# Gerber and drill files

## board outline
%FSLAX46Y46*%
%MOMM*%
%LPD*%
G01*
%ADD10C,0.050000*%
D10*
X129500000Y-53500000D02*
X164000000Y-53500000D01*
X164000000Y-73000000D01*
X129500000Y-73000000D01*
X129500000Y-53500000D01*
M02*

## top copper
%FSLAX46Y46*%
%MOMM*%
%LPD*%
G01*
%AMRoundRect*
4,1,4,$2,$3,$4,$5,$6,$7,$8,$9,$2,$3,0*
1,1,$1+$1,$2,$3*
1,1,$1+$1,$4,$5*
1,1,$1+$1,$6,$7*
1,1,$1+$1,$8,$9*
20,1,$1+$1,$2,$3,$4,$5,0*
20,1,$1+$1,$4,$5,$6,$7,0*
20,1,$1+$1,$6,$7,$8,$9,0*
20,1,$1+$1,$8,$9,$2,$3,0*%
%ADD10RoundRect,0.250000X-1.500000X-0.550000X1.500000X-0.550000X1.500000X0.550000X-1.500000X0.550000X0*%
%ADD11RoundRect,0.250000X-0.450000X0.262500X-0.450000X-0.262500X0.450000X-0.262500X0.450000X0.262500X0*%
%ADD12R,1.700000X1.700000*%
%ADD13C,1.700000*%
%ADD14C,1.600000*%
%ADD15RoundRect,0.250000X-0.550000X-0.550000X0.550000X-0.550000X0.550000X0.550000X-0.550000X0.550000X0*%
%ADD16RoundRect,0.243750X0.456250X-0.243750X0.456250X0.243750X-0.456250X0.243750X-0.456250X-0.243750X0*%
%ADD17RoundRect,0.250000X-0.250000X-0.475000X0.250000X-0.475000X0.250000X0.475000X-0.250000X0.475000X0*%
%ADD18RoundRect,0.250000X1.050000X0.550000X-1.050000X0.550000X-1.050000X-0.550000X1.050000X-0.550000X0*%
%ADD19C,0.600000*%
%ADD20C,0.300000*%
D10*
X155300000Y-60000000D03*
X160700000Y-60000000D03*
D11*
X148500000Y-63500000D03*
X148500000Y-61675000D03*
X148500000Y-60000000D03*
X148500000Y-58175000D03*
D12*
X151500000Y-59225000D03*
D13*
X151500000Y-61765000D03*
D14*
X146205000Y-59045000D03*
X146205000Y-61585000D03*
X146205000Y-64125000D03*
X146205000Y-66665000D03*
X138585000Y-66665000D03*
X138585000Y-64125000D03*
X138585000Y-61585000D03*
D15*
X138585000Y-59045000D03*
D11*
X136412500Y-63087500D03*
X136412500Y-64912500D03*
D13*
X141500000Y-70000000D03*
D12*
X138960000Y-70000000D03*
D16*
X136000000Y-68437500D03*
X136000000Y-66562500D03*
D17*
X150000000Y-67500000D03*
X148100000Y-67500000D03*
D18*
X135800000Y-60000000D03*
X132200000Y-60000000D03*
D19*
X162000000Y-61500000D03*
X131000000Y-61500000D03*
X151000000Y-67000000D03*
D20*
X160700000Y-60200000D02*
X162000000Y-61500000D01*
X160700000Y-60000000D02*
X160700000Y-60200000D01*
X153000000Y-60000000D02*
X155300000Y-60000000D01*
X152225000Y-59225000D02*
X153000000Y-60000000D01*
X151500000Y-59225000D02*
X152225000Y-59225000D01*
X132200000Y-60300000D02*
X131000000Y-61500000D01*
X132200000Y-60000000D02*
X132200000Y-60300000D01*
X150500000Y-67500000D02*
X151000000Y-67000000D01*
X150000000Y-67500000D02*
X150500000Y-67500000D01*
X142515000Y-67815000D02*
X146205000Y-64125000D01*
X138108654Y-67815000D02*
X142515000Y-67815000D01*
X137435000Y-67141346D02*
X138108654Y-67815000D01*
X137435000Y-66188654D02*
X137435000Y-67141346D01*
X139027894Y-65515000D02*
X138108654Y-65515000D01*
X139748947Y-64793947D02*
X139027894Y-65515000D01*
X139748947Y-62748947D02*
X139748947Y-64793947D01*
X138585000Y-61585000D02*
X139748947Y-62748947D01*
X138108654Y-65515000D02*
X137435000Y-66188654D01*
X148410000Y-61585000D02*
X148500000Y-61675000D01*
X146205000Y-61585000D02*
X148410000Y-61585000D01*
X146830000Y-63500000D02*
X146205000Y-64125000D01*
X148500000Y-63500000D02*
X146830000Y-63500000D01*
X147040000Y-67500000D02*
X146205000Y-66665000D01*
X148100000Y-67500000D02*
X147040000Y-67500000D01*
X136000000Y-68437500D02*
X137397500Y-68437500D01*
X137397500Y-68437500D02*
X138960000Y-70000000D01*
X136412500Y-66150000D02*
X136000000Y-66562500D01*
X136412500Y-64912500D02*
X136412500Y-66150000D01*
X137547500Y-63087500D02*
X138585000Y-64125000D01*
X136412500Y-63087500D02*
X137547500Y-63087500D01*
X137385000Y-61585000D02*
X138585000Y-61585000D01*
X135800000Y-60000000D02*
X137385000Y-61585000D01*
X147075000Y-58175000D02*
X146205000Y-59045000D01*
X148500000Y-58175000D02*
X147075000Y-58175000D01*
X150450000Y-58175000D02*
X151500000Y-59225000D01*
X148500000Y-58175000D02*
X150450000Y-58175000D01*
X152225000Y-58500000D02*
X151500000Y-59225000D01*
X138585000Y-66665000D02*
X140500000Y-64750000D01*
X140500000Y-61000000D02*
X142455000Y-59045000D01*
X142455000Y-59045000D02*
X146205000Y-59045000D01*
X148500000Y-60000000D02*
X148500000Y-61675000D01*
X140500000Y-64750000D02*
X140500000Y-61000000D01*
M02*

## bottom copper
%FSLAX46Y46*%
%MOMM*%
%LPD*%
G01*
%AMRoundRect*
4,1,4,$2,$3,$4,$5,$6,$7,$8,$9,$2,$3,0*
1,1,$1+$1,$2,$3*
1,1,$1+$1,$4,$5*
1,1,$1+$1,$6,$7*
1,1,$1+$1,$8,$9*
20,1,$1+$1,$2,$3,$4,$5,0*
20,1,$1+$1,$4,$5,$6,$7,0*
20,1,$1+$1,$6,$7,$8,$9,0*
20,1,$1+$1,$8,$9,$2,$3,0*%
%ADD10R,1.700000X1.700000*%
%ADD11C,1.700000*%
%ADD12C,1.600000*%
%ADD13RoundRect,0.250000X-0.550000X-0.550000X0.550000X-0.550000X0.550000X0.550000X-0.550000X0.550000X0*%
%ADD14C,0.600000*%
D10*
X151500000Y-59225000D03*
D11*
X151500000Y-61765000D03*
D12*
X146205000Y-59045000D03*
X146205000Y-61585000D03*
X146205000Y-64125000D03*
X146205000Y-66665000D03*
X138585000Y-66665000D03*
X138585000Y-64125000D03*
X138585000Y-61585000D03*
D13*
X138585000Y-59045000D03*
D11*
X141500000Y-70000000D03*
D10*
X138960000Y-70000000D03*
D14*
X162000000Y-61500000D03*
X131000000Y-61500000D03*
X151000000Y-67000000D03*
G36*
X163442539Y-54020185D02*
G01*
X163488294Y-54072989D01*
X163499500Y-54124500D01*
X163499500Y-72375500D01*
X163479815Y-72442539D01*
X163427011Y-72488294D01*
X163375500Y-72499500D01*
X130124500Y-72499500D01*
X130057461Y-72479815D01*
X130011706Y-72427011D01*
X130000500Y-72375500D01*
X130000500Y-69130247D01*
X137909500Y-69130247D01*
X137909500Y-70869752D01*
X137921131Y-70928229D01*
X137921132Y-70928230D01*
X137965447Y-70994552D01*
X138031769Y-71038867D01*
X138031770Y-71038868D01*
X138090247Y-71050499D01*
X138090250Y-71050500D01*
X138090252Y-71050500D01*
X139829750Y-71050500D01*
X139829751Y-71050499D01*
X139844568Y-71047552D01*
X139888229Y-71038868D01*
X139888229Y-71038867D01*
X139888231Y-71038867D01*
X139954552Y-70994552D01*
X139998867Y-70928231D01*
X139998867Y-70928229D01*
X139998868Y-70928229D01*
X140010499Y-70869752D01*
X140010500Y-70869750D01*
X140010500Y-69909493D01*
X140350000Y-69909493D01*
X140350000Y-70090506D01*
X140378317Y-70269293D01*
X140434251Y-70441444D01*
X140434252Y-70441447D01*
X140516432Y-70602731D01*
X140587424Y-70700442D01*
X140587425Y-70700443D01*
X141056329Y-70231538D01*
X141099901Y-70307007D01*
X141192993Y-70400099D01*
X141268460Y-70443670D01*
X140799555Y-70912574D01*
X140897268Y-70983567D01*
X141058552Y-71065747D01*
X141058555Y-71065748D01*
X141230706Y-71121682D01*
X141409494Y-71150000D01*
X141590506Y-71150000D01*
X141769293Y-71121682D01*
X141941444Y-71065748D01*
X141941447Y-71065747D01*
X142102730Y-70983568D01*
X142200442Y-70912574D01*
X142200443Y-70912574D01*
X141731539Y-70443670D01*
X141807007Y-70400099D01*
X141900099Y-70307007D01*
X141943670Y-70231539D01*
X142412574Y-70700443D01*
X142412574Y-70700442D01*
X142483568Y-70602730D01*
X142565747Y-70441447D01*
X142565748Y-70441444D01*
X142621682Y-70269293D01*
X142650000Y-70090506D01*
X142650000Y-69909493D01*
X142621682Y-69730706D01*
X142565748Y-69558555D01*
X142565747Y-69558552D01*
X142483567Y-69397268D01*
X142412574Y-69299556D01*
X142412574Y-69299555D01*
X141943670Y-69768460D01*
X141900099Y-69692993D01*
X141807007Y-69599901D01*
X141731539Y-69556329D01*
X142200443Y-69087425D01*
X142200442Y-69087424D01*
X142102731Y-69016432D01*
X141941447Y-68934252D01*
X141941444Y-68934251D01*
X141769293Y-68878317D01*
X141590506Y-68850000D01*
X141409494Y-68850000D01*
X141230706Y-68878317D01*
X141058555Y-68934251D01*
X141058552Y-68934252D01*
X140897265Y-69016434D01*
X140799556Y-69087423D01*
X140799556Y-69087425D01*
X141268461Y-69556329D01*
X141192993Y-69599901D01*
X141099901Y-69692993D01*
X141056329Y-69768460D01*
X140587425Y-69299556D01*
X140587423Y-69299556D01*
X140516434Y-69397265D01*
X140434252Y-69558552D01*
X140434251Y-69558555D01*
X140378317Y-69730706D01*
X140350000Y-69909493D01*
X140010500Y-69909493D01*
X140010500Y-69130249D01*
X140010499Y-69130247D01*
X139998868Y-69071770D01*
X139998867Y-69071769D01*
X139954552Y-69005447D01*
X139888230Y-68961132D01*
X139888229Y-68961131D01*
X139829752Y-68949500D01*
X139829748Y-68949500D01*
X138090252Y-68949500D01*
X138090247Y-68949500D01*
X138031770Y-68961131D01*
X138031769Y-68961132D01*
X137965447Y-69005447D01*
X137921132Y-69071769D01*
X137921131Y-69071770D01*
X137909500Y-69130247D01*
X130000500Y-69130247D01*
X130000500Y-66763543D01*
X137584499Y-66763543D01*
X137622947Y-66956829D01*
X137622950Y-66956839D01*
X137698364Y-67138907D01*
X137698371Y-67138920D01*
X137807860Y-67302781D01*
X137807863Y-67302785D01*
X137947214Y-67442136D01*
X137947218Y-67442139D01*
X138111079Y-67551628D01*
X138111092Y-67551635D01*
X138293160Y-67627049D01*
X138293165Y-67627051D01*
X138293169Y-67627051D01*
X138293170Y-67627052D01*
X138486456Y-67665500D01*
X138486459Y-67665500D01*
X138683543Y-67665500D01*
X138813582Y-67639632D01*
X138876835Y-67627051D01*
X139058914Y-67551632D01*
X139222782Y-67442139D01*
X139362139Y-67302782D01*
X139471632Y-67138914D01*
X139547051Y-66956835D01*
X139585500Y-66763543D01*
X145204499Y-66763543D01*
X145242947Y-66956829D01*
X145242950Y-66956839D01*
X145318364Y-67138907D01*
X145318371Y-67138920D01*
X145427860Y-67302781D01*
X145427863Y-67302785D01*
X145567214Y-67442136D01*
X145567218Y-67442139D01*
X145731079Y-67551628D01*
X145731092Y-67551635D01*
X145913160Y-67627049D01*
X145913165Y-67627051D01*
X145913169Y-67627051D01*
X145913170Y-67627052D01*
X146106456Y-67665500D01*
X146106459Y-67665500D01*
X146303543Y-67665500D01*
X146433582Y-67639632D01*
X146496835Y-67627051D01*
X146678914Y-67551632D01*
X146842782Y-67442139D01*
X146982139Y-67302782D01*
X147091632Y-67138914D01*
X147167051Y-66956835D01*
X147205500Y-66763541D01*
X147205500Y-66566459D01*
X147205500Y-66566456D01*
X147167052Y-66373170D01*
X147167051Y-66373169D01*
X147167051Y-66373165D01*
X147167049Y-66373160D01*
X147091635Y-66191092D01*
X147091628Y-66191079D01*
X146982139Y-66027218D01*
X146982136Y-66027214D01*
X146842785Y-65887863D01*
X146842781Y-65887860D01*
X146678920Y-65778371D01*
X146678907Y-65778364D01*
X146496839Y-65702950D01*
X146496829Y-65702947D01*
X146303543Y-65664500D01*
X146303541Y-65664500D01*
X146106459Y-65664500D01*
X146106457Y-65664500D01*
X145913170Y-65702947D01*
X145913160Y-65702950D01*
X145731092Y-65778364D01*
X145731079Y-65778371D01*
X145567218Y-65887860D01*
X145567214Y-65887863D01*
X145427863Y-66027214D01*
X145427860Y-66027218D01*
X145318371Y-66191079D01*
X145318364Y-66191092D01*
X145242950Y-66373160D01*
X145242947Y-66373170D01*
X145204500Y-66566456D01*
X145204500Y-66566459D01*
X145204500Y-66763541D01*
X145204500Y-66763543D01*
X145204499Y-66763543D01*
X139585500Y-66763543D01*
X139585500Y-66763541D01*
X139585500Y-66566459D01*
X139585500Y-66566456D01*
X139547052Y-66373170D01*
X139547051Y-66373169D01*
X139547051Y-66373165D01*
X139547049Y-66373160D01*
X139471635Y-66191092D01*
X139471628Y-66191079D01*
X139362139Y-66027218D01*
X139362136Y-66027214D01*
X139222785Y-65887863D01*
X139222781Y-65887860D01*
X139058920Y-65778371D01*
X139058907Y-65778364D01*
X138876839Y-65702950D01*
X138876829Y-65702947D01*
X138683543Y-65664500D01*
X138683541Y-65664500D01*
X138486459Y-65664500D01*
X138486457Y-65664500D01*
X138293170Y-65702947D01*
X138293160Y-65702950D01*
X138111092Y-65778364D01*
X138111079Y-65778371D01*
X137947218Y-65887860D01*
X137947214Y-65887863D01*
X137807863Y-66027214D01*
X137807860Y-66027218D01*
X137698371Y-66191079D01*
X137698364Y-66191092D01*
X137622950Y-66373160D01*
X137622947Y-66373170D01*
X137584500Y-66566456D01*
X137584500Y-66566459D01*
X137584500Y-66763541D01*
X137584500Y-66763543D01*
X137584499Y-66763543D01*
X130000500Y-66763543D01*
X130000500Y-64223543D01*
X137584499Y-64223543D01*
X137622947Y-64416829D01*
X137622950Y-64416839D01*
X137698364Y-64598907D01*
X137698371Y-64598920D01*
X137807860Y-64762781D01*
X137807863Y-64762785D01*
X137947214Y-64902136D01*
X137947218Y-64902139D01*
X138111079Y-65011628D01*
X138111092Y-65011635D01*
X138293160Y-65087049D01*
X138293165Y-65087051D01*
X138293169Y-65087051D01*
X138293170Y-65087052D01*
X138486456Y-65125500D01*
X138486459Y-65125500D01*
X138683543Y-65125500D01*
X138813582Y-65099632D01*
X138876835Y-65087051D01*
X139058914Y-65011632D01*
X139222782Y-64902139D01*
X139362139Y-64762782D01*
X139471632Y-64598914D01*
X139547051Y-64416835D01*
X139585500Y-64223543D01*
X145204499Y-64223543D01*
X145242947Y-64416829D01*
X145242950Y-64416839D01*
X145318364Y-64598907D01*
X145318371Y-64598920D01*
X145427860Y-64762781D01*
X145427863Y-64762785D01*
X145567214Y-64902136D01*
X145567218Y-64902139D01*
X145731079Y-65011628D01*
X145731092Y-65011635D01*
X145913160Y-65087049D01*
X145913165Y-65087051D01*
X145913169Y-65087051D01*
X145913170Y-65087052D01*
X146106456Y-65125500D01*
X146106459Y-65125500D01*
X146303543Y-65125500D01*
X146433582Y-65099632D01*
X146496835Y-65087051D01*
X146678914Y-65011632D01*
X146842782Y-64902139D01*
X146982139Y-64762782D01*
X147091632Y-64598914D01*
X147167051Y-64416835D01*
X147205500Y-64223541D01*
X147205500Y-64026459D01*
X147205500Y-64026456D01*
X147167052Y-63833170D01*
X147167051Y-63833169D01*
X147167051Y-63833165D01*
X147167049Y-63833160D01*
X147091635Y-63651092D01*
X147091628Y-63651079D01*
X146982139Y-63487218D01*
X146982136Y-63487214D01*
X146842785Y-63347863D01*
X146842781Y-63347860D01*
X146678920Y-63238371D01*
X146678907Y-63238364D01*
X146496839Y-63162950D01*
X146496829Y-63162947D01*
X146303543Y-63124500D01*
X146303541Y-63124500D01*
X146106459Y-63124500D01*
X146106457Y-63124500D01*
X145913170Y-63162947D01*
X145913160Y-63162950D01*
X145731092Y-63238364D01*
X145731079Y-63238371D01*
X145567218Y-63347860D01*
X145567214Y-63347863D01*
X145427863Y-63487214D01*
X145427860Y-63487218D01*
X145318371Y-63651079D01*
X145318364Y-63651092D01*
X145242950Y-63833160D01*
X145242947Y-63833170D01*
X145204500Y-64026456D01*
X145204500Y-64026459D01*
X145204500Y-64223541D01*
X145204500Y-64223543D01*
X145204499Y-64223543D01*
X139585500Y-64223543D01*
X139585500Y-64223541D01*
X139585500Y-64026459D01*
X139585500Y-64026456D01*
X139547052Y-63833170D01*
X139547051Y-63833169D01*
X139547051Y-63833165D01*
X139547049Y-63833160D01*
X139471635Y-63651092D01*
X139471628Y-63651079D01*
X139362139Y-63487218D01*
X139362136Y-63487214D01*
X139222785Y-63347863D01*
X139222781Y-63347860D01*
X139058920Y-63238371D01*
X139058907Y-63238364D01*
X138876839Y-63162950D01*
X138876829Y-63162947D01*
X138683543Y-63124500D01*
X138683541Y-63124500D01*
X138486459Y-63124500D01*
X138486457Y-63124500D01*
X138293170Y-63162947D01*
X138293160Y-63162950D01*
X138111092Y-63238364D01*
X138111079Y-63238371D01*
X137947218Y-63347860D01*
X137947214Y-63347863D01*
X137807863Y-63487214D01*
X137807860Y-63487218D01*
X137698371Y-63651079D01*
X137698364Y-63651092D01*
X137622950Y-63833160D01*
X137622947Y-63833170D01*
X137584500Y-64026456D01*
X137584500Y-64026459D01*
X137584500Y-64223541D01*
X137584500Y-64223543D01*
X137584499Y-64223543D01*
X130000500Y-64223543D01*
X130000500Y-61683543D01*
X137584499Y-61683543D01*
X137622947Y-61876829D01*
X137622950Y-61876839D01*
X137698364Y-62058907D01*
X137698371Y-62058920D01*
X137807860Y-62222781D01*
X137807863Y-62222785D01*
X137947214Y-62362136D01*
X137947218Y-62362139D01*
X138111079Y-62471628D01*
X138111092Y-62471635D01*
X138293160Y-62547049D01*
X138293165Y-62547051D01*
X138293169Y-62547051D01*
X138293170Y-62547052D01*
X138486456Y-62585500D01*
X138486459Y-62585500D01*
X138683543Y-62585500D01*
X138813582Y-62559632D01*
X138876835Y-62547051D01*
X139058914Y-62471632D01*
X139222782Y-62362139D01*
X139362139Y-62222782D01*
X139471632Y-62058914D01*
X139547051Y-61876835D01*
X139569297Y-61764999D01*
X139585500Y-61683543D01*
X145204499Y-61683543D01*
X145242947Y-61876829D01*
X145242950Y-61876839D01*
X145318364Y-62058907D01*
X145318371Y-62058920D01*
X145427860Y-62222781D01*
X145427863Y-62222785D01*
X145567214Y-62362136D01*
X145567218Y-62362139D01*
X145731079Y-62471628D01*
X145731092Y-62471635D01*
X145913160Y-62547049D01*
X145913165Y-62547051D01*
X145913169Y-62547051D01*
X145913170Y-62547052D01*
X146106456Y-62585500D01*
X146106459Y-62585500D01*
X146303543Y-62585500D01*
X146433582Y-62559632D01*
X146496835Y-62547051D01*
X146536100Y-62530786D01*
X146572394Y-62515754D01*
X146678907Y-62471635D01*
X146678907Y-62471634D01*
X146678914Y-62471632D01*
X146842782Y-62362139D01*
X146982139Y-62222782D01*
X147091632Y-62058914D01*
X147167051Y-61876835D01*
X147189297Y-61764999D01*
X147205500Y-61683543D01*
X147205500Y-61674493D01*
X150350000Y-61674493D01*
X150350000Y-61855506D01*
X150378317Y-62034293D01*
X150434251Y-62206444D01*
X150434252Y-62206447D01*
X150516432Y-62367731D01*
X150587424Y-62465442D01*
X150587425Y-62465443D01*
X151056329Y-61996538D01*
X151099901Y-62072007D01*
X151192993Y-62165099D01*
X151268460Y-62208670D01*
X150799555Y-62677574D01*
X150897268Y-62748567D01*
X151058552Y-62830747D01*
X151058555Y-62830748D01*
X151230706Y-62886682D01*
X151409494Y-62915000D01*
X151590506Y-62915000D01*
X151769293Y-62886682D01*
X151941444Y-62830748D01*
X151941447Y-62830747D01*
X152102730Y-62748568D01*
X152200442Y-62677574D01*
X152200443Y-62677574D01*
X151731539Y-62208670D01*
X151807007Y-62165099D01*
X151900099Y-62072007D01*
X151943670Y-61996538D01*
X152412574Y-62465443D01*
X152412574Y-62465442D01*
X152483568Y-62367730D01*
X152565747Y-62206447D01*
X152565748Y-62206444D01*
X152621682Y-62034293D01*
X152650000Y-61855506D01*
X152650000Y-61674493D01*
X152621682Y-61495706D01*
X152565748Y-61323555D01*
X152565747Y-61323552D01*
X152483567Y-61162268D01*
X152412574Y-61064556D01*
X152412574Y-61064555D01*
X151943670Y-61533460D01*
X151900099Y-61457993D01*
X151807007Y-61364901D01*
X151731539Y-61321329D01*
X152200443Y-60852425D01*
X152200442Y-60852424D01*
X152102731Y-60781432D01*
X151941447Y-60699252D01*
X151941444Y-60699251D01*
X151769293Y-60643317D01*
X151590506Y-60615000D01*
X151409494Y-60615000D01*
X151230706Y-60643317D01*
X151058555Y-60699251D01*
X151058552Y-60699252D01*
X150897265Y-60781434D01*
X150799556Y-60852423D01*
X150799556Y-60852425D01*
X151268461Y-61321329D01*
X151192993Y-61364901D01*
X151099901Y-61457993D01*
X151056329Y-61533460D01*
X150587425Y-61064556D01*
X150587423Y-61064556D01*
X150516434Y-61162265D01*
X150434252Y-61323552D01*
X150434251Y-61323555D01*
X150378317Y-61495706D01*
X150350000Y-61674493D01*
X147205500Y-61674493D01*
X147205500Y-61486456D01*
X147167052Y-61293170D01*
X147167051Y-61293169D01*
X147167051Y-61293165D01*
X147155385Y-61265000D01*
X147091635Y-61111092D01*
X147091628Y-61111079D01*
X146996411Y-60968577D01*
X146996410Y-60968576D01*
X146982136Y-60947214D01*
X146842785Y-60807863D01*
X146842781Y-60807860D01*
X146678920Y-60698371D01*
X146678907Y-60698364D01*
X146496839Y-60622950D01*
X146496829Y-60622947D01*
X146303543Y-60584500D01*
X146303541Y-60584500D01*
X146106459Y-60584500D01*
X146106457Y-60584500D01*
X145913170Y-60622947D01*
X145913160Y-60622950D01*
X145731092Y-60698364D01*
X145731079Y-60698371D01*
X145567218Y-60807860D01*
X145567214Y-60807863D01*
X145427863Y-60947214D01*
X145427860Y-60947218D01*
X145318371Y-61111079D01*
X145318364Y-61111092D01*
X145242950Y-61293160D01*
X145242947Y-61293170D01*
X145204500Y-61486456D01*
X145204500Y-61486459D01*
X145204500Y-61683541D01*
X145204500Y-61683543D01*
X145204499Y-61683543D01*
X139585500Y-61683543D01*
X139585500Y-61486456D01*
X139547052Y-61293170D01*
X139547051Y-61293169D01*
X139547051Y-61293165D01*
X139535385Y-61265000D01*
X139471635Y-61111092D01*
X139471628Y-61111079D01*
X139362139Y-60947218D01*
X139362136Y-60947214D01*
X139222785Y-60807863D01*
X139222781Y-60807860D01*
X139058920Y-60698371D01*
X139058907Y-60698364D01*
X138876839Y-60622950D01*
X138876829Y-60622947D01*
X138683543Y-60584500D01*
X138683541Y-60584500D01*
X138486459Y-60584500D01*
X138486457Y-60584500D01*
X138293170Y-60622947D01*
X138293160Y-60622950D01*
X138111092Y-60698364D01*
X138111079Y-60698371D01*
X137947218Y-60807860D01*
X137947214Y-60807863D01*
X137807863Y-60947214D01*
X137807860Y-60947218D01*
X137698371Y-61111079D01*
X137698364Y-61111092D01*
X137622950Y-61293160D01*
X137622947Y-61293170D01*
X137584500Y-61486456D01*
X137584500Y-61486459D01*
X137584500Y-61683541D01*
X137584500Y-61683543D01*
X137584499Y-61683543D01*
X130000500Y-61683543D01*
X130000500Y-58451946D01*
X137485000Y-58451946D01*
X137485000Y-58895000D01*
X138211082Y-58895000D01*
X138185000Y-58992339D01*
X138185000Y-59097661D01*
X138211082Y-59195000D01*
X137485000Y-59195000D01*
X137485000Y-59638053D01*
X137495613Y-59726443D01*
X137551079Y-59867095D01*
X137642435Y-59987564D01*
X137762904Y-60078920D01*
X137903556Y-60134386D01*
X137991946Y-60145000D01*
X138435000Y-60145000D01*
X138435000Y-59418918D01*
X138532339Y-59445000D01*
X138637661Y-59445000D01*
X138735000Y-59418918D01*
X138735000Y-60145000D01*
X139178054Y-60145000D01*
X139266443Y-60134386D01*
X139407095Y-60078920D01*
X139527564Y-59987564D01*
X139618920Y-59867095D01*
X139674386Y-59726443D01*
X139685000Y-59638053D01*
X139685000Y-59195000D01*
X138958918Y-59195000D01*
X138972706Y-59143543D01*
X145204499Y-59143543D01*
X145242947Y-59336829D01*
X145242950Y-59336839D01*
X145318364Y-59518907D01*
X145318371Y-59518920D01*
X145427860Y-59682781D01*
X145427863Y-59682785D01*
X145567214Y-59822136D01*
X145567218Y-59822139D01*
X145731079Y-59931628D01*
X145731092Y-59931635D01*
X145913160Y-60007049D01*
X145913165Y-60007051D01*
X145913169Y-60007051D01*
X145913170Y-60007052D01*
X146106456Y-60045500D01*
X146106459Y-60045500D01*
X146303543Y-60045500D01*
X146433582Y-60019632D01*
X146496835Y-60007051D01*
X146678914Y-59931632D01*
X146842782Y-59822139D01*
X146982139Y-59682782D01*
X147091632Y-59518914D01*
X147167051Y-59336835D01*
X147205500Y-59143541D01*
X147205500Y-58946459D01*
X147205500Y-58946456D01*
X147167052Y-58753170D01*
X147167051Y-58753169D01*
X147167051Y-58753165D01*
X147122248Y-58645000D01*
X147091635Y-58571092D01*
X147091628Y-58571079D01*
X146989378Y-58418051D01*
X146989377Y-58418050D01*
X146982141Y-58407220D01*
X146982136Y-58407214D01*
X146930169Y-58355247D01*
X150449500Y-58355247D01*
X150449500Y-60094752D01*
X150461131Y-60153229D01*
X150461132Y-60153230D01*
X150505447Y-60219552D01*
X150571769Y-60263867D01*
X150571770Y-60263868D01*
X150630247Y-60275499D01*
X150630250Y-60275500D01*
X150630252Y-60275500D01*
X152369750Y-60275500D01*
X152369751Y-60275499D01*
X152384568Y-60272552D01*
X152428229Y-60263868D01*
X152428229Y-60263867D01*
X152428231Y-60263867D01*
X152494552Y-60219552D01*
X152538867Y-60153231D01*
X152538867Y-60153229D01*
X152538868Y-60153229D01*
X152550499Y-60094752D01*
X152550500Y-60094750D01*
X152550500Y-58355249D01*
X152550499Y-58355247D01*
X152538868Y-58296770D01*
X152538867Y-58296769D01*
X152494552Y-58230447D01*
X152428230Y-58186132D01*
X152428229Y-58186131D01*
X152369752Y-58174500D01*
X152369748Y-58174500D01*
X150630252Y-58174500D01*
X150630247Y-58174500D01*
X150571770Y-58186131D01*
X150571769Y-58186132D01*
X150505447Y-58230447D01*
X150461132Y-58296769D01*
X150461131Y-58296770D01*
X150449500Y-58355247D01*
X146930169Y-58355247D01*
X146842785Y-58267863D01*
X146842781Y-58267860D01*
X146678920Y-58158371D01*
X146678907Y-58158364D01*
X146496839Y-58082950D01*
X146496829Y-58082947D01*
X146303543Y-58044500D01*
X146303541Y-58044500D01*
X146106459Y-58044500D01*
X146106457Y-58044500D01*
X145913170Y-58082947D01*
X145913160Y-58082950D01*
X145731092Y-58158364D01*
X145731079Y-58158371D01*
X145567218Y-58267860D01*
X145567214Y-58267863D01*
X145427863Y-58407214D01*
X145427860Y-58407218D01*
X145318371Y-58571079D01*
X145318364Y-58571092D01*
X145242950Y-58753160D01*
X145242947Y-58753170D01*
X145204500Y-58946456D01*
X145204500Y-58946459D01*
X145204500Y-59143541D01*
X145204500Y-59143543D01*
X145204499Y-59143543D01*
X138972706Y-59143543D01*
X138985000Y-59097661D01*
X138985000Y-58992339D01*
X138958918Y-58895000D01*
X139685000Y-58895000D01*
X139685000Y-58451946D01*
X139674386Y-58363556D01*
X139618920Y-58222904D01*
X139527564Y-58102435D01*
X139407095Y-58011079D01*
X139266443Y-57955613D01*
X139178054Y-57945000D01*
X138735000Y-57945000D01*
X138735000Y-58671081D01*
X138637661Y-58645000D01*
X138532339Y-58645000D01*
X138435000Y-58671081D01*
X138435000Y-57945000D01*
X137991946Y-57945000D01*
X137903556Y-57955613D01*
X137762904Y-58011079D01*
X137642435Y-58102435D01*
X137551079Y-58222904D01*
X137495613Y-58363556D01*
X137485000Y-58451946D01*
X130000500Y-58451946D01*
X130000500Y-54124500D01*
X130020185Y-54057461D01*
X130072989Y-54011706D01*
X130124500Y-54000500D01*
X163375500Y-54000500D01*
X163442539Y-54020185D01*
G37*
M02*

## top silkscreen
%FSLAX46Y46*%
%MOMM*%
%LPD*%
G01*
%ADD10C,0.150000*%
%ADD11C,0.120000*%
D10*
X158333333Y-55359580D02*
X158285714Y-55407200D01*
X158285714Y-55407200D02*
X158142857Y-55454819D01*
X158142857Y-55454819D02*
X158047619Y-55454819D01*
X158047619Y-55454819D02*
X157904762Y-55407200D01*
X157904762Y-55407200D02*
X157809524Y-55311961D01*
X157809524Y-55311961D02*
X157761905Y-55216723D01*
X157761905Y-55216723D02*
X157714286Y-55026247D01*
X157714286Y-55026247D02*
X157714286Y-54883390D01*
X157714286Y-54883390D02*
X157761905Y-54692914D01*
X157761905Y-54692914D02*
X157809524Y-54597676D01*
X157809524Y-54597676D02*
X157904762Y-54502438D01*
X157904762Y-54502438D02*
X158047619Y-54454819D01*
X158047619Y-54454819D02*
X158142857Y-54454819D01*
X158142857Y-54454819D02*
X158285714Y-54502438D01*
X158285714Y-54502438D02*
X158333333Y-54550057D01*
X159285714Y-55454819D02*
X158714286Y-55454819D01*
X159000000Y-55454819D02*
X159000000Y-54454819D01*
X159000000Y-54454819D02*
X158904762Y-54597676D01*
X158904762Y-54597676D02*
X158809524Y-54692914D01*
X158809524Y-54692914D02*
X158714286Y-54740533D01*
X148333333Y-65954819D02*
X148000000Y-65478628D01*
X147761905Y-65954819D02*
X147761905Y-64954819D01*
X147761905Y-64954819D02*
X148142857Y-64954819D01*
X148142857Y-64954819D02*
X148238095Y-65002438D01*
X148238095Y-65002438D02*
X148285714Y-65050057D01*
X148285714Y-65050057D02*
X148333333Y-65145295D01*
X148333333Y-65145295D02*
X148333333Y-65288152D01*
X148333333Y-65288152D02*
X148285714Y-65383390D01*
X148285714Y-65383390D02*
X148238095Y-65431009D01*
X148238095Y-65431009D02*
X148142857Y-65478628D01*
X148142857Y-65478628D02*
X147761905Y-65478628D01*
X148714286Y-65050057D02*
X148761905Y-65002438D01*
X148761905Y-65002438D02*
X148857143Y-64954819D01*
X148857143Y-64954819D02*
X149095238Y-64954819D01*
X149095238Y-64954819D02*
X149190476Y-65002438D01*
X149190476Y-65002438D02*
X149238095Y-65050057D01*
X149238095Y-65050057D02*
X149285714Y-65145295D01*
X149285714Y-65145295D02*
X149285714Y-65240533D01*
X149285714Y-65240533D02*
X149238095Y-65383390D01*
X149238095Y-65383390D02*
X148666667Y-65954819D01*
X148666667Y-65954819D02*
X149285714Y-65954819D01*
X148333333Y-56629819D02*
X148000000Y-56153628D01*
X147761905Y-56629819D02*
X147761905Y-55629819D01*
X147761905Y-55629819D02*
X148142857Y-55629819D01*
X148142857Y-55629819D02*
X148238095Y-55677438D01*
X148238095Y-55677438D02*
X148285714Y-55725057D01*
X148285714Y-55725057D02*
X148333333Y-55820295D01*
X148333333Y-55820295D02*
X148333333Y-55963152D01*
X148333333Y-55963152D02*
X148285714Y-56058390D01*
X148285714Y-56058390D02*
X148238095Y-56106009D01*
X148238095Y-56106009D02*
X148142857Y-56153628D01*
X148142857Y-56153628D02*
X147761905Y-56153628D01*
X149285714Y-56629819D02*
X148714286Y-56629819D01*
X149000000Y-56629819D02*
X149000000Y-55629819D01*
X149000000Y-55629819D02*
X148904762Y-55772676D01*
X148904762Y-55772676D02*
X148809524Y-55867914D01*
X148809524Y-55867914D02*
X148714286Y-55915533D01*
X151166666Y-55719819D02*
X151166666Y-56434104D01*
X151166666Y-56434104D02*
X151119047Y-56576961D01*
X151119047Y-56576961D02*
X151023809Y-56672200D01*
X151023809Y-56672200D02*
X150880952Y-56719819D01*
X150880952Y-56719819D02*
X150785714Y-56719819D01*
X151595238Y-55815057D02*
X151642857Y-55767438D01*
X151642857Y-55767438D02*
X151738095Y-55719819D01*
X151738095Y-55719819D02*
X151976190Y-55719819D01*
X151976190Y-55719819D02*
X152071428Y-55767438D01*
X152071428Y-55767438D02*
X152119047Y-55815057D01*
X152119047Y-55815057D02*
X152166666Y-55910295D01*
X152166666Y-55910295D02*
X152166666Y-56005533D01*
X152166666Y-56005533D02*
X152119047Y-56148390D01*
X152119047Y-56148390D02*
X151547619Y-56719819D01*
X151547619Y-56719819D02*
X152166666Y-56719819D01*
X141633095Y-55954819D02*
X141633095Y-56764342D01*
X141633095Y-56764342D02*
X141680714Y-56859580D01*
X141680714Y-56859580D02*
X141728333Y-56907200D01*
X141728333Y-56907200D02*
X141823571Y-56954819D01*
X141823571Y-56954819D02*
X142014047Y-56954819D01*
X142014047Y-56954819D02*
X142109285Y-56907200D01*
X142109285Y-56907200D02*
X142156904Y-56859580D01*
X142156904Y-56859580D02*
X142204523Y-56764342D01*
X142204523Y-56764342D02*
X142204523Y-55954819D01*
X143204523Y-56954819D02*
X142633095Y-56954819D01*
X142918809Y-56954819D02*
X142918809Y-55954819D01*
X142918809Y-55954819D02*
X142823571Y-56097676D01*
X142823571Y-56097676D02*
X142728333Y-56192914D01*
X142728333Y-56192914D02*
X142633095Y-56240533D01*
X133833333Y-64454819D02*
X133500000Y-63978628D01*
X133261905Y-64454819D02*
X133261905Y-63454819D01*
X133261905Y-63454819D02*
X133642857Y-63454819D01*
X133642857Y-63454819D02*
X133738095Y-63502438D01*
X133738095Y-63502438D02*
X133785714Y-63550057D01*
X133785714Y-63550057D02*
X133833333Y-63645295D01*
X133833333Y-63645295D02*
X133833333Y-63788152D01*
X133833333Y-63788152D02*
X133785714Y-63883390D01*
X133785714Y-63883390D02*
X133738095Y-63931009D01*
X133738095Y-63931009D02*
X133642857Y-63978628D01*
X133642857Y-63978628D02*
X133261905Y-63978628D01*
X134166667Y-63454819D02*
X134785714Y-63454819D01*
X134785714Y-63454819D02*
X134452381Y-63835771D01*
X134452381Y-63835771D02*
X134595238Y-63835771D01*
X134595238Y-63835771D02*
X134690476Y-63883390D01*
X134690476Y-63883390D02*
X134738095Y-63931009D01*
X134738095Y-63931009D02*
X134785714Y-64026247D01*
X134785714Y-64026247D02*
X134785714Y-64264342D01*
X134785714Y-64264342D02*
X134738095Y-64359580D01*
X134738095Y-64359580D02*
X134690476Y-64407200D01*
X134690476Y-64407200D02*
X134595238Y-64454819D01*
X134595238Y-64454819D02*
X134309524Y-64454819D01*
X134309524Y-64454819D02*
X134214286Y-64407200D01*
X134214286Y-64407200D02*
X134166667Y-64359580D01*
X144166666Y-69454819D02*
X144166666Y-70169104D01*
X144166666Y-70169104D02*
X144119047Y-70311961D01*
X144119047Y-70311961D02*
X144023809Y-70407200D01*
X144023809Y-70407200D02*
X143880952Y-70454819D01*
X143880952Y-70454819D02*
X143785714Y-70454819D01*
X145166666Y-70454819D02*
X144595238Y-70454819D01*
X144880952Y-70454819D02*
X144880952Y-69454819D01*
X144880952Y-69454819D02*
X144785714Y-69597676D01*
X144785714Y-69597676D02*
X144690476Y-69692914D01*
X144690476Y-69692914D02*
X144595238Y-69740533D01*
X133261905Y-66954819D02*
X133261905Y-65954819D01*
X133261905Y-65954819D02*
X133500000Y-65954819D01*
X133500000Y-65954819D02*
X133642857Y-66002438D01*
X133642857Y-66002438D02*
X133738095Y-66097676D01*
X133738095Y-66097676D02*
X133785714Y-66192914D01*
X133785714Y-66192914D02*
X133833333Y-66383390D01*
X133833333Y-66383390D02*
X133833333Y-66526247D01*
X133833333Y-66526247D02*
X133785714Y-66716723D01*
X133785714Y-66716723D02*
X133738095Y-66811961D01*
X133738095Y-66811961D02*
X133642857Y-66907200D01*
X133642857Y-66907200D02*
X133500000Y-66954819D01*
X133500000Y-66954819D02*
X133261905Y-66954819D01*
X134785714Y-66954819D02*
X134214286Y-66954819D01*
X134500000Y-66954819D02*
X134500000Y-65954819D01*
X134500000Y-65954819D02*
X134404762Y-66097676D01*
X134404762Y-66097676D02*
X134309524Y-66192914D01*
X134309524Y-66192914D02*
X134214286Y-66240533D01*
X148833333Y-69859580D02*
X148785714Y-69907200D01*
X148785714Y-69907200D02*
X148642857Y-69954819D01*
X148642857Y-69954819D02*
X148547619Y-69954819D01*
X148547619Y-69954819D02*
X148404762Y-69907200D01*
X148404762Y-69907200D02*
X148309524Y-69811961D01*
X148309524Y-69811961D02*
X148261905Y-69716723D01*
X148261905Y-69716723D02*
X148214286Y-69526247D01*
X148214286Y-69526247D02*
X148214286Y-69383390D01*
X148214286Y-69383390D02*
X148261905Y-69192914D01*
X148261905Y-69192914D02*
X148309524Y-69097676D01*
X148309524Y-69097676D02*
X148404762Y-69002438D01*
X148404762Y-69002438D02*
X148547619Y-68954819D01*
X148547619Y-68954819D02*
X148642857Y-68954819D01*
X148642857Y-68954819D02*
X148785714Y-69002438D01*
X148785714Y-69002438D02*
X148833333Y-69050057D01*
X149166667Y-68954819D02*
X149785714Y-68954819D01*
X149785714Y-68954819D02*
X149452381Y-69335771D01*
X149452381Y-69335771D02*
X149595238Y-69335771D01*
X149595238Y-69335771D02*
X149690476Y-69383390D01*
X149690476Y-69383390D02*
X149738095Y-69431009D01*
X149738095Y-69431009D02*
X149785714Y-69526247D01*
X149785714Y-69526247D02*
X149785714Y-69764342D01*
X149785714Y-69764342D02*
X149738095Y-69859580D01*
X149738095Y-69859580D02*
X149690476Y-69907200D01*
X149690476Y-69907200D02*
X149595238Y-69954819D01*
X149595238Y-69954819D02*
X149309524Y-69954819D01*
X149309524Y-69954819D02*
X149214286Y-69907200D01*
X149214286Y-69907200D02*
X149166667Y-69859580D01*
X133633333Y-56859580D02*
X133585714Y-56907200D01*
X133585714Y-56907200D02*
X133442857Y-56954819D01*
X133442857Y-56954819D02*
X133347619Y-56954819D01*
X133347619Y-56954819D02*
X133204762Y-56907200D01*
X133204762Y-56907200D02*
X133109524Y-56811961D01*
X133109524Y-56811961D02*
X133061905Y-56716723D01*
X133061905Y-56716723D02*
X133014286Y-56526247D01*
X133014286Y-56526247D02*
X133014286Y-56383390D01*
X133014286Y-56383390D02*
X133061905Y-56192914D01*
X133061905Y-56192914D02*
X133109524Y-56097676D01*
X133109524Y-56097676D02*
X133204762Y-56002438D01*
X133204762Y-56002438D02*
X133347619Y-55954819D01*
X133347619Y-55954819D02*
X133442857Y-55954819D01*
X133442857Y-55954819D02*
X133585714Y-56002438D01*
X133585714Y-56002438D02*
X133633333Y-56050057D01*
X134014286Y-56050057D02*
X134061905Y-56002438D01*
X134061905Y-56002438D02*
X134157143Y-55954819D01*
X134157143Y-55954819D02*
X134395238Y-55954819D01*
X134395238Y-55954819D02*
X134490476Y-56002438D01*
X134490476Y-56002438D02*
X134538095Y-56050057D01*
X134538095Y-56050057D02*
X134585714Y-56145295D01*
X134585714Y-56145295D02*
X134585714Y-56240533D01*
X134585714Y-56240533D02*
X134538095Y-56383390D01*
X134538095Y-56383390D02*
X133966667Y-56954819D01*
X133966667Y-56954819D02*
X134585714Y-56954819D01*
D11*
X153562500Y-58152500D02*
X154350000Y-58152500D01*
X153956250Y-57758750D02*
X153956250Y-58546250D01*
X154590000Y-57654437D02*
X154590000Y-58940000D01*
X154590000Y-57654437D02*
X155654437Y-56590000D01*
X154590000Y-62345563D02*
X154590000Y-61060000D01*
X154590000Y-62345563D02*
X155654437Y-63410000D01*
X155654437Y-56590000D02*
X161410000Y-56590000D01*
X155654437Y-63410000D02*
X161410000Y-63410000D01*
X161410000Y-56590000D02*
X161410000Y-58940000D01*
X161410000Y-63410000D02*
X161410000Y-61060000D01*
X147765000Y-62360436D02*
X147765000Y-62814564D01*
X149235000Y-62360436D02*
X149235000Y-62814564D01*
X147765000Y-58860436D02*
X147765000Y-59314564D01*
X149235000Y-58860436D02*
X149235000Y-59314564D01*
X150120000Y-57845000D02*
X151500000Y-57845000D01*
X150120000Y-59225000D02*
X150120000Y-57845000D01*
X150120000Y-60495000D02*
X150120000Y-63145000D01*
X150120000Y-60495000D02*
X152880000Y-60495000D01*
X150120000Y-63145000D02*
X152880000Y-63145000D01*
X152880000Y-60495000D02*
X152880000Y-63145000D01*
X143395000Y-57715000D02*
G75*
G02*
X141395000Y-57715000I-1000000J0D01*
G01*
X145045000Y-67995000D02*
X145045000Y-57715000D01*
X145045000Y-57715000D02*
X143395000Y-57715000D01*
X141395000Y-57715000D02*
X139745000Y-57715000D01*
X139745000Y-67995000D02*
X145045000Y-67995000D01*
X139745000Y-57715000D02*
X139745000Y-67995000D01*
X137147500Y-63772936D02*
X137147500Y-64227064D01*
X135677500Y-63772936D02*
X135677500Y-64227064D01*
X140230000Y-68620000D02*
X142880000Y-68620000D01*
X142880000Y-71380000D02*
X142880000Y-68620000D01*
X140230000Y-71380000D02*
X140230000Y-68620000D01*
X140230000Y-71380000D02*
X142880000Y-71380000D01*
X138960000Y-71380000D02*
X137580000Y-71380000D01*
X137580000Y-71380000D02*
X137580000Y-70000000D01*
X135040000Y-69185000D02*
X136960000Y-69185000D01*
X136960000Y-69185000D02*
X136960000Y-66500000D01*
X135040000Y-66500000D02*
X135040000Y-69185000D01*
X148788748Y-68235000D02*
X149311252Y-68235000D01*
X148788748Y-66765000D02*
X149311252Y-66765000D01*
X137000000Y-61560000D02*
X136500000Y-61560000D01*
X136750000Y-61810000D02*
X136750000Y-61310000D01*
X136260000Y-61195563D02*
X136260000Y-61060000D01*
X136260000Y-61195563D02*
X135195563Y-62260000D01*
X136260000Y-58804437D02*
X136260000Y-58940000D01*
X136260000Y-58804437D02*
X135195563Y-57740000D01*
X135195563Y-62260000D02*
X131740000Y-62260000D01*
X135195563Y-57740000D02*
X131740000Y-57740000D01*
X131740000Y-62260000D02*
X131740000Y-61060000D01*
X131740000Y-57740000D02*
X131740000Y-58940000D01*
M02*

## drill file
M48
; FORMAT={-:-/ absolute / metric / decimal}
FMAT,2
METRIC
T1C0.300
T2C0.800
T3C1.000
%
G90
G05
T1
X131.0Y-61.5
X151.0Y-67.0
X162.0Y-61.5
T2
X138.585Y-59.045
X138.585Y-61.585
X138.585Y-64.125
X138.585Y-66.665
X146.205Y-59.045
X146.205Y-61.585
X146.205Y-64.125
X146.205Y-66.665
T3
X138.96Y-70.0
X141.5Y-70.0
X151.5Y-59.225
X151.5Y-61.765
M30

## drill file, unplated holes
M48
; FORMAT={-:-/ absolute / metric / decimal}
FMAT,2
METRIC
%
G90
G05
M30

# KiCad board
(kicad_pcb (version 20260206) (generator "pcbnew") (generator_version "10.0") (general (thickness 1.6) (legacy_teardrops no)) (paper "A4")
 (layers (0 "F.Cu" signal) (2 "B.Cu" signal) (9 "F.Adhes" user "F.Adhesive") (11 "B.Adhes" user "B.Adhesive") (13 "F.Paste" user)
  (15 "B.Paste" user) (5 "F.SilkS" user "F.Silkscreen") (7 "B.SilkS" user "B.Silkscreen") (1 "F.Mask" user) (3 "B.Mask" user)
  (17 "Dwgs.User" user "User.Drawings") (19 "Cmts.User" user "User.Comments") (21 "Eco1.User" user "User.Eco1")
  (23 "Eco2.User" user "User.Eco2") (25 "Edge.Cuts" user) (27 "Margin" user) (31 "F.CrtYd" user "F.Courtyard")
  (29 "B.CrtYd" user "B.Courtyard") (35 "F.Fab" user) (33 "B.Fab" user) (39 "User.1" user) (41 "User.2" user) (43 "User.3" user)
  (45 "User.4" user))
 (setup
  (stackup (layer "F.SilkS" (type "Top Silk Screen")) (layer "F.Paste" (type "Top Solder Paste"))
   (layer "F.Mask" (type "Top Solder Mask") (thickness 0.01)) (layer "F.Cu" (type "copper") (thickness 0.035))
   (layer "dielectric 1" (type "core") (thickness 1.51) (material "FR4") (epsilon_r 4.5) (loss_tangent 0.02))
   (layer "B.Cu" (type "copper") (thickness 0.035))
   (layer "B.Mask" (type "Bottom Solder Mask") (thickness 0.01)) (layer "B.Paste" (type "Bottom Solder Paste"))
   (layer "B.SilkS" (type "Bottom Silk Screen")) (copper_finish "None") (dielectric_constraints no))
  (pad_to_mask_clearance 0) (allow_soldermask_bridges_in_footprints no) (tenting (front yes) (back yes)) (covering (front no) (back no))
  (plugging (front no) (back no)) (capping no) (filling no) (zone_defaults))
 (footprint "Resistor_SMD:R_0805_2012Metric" (layer "F.Cu") (at 136.4125 64 -90)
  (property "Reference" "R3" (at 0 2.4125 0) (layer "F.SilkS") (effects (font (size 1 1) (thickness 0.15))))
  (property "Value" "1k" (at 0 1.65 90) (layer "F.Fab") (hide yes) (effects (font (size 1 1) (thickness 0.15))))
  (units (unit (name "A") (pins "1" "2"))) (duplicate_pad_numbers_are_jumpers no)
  (fp_line (start -0.227064 0.735) (end 0.227064 0.735) (stroke (width 0.12) (type solid)) (layer "F.SilkS"))
  (fp_line (start -0.227064 -0.735) (end 0.227064 -0.735) (stroke (width 0.12) (type solid)) (layer "F.SilkS"))
  (pad "1" smd roundrect (at -0.9125 0 270) (size 1.025 1.4) (layers "F.Cu" "F.Mask" "F.Paste") (roundrect_rratio 0.243902)
   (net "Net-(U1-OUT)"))
  (pad "2" smd roundrect (at 0.9125 0 270) (size 1.025 1.4) (layers "F.Cu" "F.Mask" "F.Paste") (roundrect_rratio 0.243902)
   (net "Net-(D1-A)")))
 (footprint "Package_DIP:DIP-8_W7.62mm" (layer "F.Cu") (at 138.585 59.045)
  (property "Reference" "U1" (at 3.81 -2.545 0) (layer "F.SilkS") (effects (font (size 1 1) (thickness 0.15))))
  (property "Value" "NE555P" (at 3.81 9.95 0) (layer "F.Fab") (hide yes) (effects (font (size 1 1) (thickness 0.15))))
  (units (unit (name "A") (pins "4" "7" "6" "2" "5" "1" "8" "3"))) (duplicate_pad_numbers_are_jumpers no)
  (fp_line (start 1.16 -1.33) (end 1.16 8.95) (stroke (width 0.12) (type solid)) (layer "F.SilkS"))
  (fp_line (start 1.16 8.95) (end 6.46 8.95) (stroke (width 0.12) (type solid)) (layer "F.SilkS"))
  (fp_line (start 2.81 -1.33) (end 1.16 -1.33) (stroke (width 0.12) (type solid)) (layer "F.SilkS"))
  (fp_line (start 6.46 -1.33) (end 4.81 -1.33) (stroke (width 0.12) (type solid)) (layer "F.SilkS"))
  (fp_line (start 6.46 8.95) (end 6.46 -1.33) (stroke (width 0.12) (type solid)) (layer "F.SilkS"))
  (fp_arc (start 4.81 -1.33) (mid 3.81 -0.33) (end 2.81 -1.33) (stroke (width 0.12) (type solid)) (layer "F.SilkS"))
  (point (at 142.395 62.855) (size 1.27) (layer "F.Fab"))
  (pad "1" thru_hole roundrect (at 0 0) (size 1.6 1.6) (drill 0.8) (layers "*.Cu" "*.Mask") (remove_unused_layers no)
   (roundrect_rratio 0.15625) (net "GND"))
  (pad "2" thru_hole circle (at 0 2.54) (size 1.6 1.6) (drill 0.8) (layers "*.Cu" "*.Mask") (remove_unused_layers no) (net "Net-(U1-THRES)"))
  (pad "3" thru_hole circle (at 0 5.08) (size 1.6 1.6) (drill 0.8) (layers "*.Cu" "*.Mask") (remove_unused_layers no) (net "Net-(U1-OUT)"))
  (pad "4" thru_hole circle (at 0 7.62) (size 1.6 1.6) (drill 0.8) (layers "*.Cu" "*.Mask") (remove_unused_layers no) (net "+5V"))
  (pad "5" thru_hole circle (at 7.62 7.62) (size 1.6 1.6) (drill 0.8) (layers "*.Cu" "*.Mask") (remove_unused_layers no)
   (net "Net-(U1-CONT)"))
  (pad "6" thru_hole circle (at 7.62 5.08) (size 1.6 1.6) (drill 0.8) (layers "*.Cu" "*.Mask") (remove_unused_layers no)
   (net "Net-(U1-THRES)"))
  (pad "7" thru_hole circle (at 7.62 2.54) (size 1.6 1.6) (drill 0.8) (layers "*.Cu" "*.Mask") (remove_unused_layers no)
   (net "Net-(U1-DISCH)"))
  (pad "8" thru_hole circle (at 7.62 0) (size 1.6 1.6) (drill 0.8) (layers "*.Cu" "*.Mask") (remove_unused_layers no) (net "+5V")))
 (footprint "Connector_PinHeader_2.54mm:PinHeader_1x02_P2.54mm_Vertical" (layer "F.Cu") (at 138.96 70 90)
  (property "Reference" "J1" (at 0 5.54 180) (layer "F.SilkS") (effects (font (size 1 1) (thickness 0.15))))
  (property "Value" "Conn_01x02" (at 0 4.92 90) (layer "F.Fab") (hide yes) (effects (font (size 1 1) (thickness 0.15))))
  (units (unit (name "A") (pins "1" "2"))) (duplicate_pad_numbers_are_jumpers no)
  (fp_line (start -1.38 -1.38) (end 0 -1.38) (stroke (width 0.12) (type solid)) (layer "F.SilkS"))
  (fp_line (start -1.38 0) (end -1.38 -1.38) (stroke (width 0.12) (type solid)) (layer "F.SilkS"))
  (fp_line (start 1.38 1.27) (end 1.38 3.92) (stroke (width 0.12) (type solid)) (layer "F.SilkS"))
  (fp_line (start -1.38 1.27) (end 1.38 1.27) (stroke (width 0.12) (type solid)) (layer "F.SilkS"))
  (fp_line (start -1.38 1.27) (end -1.38 3.92) (stroke (width 0.12) (type solid)) (layer "F.SilkS"))
  (fp_line (start -1.38 3.92) (end 1.38 3.92) (stroke (width 0.12) (type solid)) (layer "F.SilkS"))
  (pad "1" thru_hole rect (at 0 0 90) (size 1.7 1.7) (drill 1) (layers "*.Cu" "*.Mask") (remove_unused_layers no) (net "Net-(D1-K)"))
  (pad "2" thru_hole circle (at 0 2.54 90) (size 1.7 1.7) (drill 1) (layers "*.Cu" "*.Mask") (remove_unused_layers no) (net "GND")))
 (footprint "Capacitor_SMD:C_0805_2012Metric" (layer "F.Cu") (at 149.05 67.5)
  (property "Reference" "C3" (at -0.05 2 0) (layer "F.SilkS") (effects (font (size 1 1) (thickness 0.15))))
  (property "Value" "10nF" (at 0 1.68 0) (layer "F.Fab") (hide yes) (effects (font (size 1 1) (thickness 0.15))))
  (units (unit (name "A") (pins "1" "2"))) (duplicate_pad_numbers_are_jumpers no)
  (fp_line (start -0.261252 -0.735) (end 0.261252 -0.735) (stroke (width 0.12) (type solid)) (layer "F.SilkS"))
  (fp_line (start -0.261252 0.735) (end 0.261252 0.735) (stroke (width 0.12) (type solid)) (layer "F.SilkS"))
  (pad "1" smd roundrect (at -0.95 0) (size 1 1.45) (layers "F.Cu" "F.Mask" "F.Paste") (roundrect_rratio 0.25) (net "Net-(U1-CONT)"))
  (pad "2" smd roundrect (at 0.95 0) (size 1 1.45) (layers "F.Cu" "F.Mask" "F.Paste") (roundrect_rratio 0.25) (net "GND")))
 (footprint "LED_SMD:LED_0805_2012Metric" (layer "F.Cu") (at 136 67.5 90)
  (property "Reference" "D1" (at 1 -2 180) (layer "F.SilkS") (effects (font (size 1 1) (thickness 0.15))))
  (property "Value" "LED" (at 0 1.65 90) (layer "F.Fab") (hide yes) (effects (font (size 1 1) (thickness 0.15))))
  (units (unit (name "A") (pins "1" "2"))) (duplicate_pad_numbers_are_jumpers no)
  (fp_line (start 1 -0.96) (end -1.685 -0.96) (stroke (width 0.12) (type solid)) (layer "F.SilkS"))
  (fp_line (start -1.685 -0.96) (end -1.685 0.96) (stroke (width 0.12) (type solid)) (layer "F.SilkS"))
  (fp_line (start -1.685 0.96) (end 1 0.96) (stroke (width 0.12) (type solid)) (layer "F.SilkS"))
  (pad "1" smd roundrect (at -0.9375 0 90) (size 0.975 1.4) (layers "F.Cu" "F.Mask" "F.Paste") (roundrect_rratio 0.25) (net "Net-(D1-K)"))
  (pad "2" smd roundrect (at 0.9375 0 90) (size 0.975 1.4) (layers "F.Cu" "F.Mask" "F.Paste") (roundrect_rratio 0.25) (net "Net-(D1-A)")))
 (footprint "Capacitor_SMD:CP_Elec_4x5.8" (layer "F.Cu") (at 134 60 180)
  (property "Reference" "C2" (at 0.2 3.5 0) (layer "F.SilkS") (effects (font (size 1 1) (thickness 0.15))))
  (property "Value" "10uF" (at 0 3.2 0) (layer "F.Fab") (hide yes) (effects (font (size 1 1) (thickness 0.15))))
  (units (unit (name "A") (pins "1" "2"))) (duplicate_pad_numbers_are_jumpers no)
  (fp_line (start 2.26 2.26) (end 2.26 1.06) (stroke (width 0.12) (type solid)) (layer "F.SilkS"))
  (fp_line (start 2.26 -2.26) (end 2.26 -1.06) (stroke (width 0.12) (type solid)) (layer "F.SilkS"))
  (fp_line (start -1.195563 2.26) (end 2.26 2.26) (stroke (width 0.12) (type solid)) (layer "F.SilkS"))
  (fp_line (start -1.195563 -2.26) (end 2.26 -2.26) (stroke (width 0.12) (type solid)) (layer "F.SilkS"))
  (fp_line (start -2.26 1.195563) (end -1.195563 2.26) (stroke (width 0.12) (type solid)) (layer "F.SilkS"))
  (fp_line (start -2.26 1.195563) (end -2.26 1.06) (stroke (width 0.12) (type solid)) (layer "F.SilkS"))
  (fp_line (start -2.26 -1.195563) (end -1.195563 -2.26) (stroke (width 0.12) (type solid)) (layer "F.SilkS"))
  (fp_line (start -2.26 -1.195563) (end -2.26 -1.06) (stroke (width 0.12) (type solid)) (layer "F.SilkS"))
  (fp_line (start -2.75 -1.81) (end -2.75 -1.31) (stroke (width 0.12) (type solid)) (layer "F.SilkS"))
  (fp_line (start -3 -1.56) (end -2.5 -1.56) (stroke (width 0.12) (type solid)) (layer "F.SilkS"))
  (pad "1" smd roundrect (at -1.8 0 180) (size 2.6 1.6) (layers "F.Cu" "F.Mask" "F.Paste") (roundrect_rratio 0.15625) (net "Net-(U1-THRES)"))
  (pad "2" smd roundrect (at 1.8 0 180) (size 2.6 1.6) (layers "F.Cu" "F.Mask" "F.Paste") (roundrect_rratio 0.15625) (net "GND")))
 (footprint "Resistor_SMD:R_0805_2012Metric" (layer "F.Cu") (at 148.5 62.5875 -90)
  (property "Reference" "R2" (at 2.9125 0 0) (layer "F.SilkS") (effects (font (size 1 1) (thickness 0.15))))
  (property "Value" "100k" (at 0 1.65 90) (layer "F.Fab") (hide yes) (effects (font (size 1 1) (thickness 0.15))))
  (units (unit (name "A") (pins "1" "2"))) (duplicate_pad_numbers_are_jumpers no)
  (fp_line (start -0.227064 0.735) (end 0.227064 0.735) (stroke (width 0.12) (type solid)) (layer "F.SilkS"))
  (fp_line (start -0.227064 -0.735) (end 0.227064 -0.735) (stroke (width 0.12) (type solid)) (layer "F.SilkS"))
  (pad "1" smd roundrect (at -0.9125 0 270) (size 1.025 1.4) (layers "F.Cu" "F.Mask" "F.Paste") (roundrect_rratio 0.243902)
   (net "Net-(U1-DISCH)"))
  (pad "2" smd roundrect (at 0.9125 0 270) (size 1.025 1.4) (layers "F.Cu" "F.Mask" "F.Paste") (roundrect_rratio 0.243902)
   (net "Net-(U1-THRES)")))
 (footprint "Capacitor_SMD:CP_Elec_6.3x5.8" (layer "F.Cu") (at 158 60)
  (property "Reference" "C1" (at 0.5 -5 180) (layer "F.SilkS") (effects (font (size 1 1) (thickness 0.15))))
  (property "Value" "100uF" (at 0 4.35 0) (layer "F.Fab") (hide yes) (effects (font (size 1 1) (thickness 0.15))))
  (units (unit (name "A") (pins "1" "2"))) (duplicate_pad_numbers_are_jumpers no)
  (fp_line (start -4.4375 -1.8475) (end -3.65 -1.8475) (stroke (width 0.12) (type solid)) (layer "F.SilkS"))
  (fp_line (start -4.04375 -2.24125) (end -4.04375 -1.45375) (stroke (width 0.12) (type solid)) (layer "F.SilkS"))
  (fp_line (start -3.41 -2.345563) (end -3.41 -1.06) (stroke (width 0.12) (type solid)) (layer "F.SilkS"))
  (fp_line (start -3.41 -2.345563) (end -2.345563 -3.41) (stroke (width 0.12) (type solid)) (layer "F.SilkS"))
  (fp_line (start -3.41 2.345563) (end -3.41 1.06) (stroke (width 0.12) (type solid)) (layer "F.SilkS"))
  (fp_line (start -3.41 2.345563) (end -2.345563 3.41) (stroke (width 0.12) (type solid)) (layer "F.SilkS"))
  (fp_line (start -2.345563 -3.41) (end 3.41 -3.41) (stroke (width 0.12) (type solid)) (layer "F.SilkS"))
  (fp_line (start -2.345563 3.41) (end 3.41 3.41) (stroke (width 0.12) (type solid)) (layer "F.SilkS"))
  (fp_line (start 3.41 -3.41) (end 3.41 -1.06) (stroke (width 0.12) (type solid)) (layer "F.SilkS"))
  (fp_line (start 3.41 3.41) (end 3.41 1.06) (stroke (width 0.12) (type solid)) (layer "F.SilkS"))
  (pad "1" smd roundrect (at -2.7 0) (size 3.5 1.6) (layers "F.Cu" "F.Mask" "F.Paste") (roundrect_rratio 0.15625) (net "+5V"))
  (pad "2" smd roundrect (at 2.7 0) (size 3.5 1.6) (layers "F.Cu" "F.Mask" "F.Paste") (roundrect_rratio 0.15625) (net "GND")))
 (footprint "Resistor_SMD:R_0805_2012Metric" (layer "F.Cu") (at 148.5 59.0875 -90)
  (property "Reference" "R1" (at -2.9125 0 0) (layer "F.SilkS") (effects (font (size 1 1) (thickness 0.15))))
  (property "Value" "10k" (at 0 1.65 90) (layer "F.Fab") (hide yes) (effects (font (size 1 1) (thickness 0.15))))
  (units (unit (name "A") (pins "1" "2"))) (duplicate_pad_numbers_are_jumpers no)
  (fp_line (start -0.227064 0.735) (end 0.227064 0.735) (stroke (width 0.12) (type solid)) (layer "F.SilkS"))
  (fp_line (start -0.227064 -0.735) (end 0.227064 -0.735) (stroke (width 0.12) (type solid)) (layer "F.SilkS"))
  (pad "1" smd roundrect (at -0.9125 0 270) (size 1.025 1.4) (layers "F.Cu" "F.Mask" "F.Paste") (roundrect_rratio 0.243902) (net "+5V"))
  (pad "2" smd roundrect (at 0.9125 0 270) (size 1.025 1.4) (layers "F.Cu" "F.Mask" "F.Paste") (roundrect_rratio 0.243902)
   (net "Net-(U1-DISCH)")))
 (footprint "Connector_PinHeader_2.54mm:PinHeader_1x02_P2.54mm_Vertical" (layer "F.Cu") (at 151.5 59.225)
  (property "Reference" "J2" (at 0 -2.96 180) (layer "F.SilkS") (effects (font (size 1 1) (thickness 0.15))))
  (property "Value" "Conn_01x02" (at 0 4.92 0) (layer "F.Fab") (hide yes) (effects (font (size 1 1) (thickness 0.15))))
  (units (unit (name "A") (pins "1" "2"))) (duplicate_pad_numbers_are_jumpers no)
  (fp_line (start -1.38 -1.38) (end 0 -1.38) (stroke (width 0.12) (type solid)) (layer "F.SilkS"))
  (fp_line (start -1.38 0) (end -1.38 -1.38) (stroke (width 0.12) (type solid)) (layer "F.SilkS"))
  (fp_line (start -1.38 1.27) (end -1.38 3.92) (stroke (width 0.12) (type solid)) (layer "F.SilkS"))
  (fp_line (start -1.38 1.27) (end 1.38 1.27) (stroke (width 0.12) (type solid)) (layer "F.SilkS"))
  (fp_line (start -1.38 3.92) (end 1.38 3.92) (stroke (width 0.12) (type solid)) (layer "F.SilkS"))
  (fp_line (start 1.38 1.27) (end 1.38 3.92) (stroke (width 0.12) (type solid)) (layer "F.SilkS"))
  (pad "1" thru_hole rect (at 0 0) (size 1.7 1.7) (drill 1) (layers "*.Cu" "*.Mask") (remove_unused_layers no) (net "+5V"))
  (pad "2" thru_hole circle (at 0 2.54) (size 1.7 1.7) (drill 1) (layers "*.Cu" "*.Mask") (remove_unused_layers no) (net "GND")))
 (gr_rect (start 129.5 53.5) (end 164 73) (stroke (width 0.05) (type default)) (fill no) (layer "Edge.Cuts"))
 (segment (start 153 60) (end 155.3 60) (width 0.3) (layer "F.Cu") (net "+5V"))
 (segment (start 147.075 58.175) (end 146.205 59.045) (width 0.3) (layer "F.Cu") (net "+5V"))
 (segment (start 148.5 58.175) (end 147.075 58.175) (width 0.3) (layer "F.Cu") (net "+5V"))
 (segment (start 148.5 58.175) (end 150.45 58.175) (width 0.3) (layer "F.Cu") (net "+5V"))
 (segment (start 152.225 59.225) (end 153 60) (width 0.3) (layer "F.Cu") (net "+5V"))
 (segment (start 140.5 64.75) (end 140.5 61) (width 0.3) (layer "F.Cu") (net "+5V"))
 (segment (start 151.5 59.225) (end 152.225 59.225) (width 0.3) (layer "F.Cu") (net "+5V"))
 (segment (start 142.455 59.045) (end 146.205 59.045) (width 0.3) (layer "F.Cu") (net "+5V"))
 (segment (start 150.45 58.175) (end 151.5 59.225) (width 0.3) (layer "F.Cu") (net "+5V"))
 (segment (start 152.225 58.5) (end 151.5 59.225) (width 0.3) (layer "F.Cu") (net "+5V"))
 (segment (start 140.5 61) (end 142.455 59.045) (width 0.3) (layer "F.Cu") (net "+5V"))
 (segment (start 138.585 66.665) (end 140.5 64.75) (width 0.3) (layer "F.Cu") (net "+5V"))
 (segment (start 132.2 60.3) (end 131 61.5) (width 0.3) (layer "F.Cu") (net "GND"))
 (segment (start 160.7 60.2) (end 162 61.5) (width 0.3) (layer "F.Cu") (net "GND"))
 (segment (start 132.2 60) (end 132.2 60.3) (width 0.3) (layer "F.Cu") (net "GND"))
 (segment (start 150 67.5) (end 150.5 67.5) (width 0.3) (layer "F.Cu") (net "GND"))
 (segment (start 150.5 67.5) (end 151 67) (width 0.3) (layer "F.Cu") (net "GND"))
 (segment (start 160.7 60) (end 160.7 60.2) (width 0.3) (layer "F.Cu") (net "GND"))
 (via (at 151 67) (size 0.6) (drill 0.3) (layers "F.Cu" "B.Cu") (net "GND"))
 (via (at 162 61.5) (size 0.6) (drill 0.3) (layers "F.Cu" "B.Cu") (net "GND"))
 (via (at 131 61.5) (size 0.6) (drill 0.3) (layers "F.Cu" "B.Cu") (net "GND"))
 (segment (start 139.748947 62.748947) (end 139.748947 64.793947) (width 0.3) (layer "F.Cu") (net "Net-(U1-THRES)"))
 (segment (start 142.515 67.815) (end 146.205 64.125) (width 0.3) (layer "F.Cu") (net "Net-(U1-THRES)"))
 (segment (start 138.108654 65.515) (end 137.435 66.188654) (width 0.3) (layer "F.Cu") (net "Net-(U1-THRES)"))
 (segment (start 139.027894 65.515) (end 138.108654 65.515) (width 0.3) (layer "F.Cu") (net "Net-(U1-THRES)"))
 (segment (start 137.435 66.188654) (end 137.435 67.141346) (width 0.3) (layer "F.Cu") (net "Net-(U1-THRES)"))
 (segment (start 137.385 61.585) (end 138.585 61.585) (width 0.3) (layer "F.Cu") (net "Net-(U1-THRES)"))
 (segment (start 139.748947 64.793947) (end 139.027894 65.515) (width 0.3) (layer "F.Cu") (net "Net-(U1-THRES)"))
 (segment (start 146.83 63.5) (end 146.205 64.125) (width 0.3) (layer "F.Cu") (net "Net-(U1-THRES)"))
 (segment (start 135.8 60) (end 137.385 61.585) (width 0.3) (layer "F.Cu") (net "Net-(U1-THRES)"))
 (segment (start 138.108654 67.815) (end 142.515 67.815) (width 0.3) (layer "F.Cu") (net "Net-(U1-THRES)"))
 (segment (start 138.585 61.585) (end 139.748947 62.748947) (width 0.3) (layer "F.Cu") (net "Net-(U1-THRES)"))
 (segment (start 137.435 67.141346) (end 138.108654 67.815) (width 0.3) (layer "F.Cu") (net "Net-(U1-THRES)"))
 (segment (start 148.5 63.5) (end 146.83 63.5) (width 0.3) (layer "F.Cu") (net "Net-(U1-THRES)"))
 (segment (start 147.04 67.5) (end 146.205 66.665) (width 0.3) (layer "F.Cu") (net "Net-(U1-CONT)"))
 (segment (start 148.1 67.5) (end 147.04 67.5) (width 0.3) (layer "F.Cu") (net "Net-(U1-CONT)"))
 (segment (start 136.4125 66.15) (end 136 66.5625) (width 0.3) (layer "F.Cu") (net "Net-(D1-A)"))
 (segment (start 136.4125 64.9125) (end 136.4125 66.15) (width 0.3) (layer "F.Cu") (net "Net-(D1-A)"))
 (segment (start 136 68.4375) (end 137.3975 68.4375) (width 0.3) (layer "F.Cu") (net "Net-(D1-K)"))
 (segment (start 137.3975 68.4375) (end 138.96 70) (width 0.3) (layer "F.Cu") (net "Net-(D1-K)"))
 (segment (start 148.41 61.585) (end 148.5 61.675) (width 0.3) (layer "F.Cu") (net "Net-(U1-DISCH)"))
 (segment (start 146.205 61.585) (end 148.41 61.585) (width 0.3) (layer "F.Cu") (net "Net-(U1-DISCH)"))
 (segment (start 148.5 60) (end 148.5 61.675) (width 0.3) (layer "F.Cu") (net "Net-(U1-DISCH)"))
 (segment (start 137.5475 63.0875) (end 138.585 64.125) (width 0.3) (layer "F.Cu") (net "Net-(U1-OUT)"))
 (segment (start 136.4125 63.0875) (end 137.5475 63.0875) (width 0.3) (layer "F.Cu") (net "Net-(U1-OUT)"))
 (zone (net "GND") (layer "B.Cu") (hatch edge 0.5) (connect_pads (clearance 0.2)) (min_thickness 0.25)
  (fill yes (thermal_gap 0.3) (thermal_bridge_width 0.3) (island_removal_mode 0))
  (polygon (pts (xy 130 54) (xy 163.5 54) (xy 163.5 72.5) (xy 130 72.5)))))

